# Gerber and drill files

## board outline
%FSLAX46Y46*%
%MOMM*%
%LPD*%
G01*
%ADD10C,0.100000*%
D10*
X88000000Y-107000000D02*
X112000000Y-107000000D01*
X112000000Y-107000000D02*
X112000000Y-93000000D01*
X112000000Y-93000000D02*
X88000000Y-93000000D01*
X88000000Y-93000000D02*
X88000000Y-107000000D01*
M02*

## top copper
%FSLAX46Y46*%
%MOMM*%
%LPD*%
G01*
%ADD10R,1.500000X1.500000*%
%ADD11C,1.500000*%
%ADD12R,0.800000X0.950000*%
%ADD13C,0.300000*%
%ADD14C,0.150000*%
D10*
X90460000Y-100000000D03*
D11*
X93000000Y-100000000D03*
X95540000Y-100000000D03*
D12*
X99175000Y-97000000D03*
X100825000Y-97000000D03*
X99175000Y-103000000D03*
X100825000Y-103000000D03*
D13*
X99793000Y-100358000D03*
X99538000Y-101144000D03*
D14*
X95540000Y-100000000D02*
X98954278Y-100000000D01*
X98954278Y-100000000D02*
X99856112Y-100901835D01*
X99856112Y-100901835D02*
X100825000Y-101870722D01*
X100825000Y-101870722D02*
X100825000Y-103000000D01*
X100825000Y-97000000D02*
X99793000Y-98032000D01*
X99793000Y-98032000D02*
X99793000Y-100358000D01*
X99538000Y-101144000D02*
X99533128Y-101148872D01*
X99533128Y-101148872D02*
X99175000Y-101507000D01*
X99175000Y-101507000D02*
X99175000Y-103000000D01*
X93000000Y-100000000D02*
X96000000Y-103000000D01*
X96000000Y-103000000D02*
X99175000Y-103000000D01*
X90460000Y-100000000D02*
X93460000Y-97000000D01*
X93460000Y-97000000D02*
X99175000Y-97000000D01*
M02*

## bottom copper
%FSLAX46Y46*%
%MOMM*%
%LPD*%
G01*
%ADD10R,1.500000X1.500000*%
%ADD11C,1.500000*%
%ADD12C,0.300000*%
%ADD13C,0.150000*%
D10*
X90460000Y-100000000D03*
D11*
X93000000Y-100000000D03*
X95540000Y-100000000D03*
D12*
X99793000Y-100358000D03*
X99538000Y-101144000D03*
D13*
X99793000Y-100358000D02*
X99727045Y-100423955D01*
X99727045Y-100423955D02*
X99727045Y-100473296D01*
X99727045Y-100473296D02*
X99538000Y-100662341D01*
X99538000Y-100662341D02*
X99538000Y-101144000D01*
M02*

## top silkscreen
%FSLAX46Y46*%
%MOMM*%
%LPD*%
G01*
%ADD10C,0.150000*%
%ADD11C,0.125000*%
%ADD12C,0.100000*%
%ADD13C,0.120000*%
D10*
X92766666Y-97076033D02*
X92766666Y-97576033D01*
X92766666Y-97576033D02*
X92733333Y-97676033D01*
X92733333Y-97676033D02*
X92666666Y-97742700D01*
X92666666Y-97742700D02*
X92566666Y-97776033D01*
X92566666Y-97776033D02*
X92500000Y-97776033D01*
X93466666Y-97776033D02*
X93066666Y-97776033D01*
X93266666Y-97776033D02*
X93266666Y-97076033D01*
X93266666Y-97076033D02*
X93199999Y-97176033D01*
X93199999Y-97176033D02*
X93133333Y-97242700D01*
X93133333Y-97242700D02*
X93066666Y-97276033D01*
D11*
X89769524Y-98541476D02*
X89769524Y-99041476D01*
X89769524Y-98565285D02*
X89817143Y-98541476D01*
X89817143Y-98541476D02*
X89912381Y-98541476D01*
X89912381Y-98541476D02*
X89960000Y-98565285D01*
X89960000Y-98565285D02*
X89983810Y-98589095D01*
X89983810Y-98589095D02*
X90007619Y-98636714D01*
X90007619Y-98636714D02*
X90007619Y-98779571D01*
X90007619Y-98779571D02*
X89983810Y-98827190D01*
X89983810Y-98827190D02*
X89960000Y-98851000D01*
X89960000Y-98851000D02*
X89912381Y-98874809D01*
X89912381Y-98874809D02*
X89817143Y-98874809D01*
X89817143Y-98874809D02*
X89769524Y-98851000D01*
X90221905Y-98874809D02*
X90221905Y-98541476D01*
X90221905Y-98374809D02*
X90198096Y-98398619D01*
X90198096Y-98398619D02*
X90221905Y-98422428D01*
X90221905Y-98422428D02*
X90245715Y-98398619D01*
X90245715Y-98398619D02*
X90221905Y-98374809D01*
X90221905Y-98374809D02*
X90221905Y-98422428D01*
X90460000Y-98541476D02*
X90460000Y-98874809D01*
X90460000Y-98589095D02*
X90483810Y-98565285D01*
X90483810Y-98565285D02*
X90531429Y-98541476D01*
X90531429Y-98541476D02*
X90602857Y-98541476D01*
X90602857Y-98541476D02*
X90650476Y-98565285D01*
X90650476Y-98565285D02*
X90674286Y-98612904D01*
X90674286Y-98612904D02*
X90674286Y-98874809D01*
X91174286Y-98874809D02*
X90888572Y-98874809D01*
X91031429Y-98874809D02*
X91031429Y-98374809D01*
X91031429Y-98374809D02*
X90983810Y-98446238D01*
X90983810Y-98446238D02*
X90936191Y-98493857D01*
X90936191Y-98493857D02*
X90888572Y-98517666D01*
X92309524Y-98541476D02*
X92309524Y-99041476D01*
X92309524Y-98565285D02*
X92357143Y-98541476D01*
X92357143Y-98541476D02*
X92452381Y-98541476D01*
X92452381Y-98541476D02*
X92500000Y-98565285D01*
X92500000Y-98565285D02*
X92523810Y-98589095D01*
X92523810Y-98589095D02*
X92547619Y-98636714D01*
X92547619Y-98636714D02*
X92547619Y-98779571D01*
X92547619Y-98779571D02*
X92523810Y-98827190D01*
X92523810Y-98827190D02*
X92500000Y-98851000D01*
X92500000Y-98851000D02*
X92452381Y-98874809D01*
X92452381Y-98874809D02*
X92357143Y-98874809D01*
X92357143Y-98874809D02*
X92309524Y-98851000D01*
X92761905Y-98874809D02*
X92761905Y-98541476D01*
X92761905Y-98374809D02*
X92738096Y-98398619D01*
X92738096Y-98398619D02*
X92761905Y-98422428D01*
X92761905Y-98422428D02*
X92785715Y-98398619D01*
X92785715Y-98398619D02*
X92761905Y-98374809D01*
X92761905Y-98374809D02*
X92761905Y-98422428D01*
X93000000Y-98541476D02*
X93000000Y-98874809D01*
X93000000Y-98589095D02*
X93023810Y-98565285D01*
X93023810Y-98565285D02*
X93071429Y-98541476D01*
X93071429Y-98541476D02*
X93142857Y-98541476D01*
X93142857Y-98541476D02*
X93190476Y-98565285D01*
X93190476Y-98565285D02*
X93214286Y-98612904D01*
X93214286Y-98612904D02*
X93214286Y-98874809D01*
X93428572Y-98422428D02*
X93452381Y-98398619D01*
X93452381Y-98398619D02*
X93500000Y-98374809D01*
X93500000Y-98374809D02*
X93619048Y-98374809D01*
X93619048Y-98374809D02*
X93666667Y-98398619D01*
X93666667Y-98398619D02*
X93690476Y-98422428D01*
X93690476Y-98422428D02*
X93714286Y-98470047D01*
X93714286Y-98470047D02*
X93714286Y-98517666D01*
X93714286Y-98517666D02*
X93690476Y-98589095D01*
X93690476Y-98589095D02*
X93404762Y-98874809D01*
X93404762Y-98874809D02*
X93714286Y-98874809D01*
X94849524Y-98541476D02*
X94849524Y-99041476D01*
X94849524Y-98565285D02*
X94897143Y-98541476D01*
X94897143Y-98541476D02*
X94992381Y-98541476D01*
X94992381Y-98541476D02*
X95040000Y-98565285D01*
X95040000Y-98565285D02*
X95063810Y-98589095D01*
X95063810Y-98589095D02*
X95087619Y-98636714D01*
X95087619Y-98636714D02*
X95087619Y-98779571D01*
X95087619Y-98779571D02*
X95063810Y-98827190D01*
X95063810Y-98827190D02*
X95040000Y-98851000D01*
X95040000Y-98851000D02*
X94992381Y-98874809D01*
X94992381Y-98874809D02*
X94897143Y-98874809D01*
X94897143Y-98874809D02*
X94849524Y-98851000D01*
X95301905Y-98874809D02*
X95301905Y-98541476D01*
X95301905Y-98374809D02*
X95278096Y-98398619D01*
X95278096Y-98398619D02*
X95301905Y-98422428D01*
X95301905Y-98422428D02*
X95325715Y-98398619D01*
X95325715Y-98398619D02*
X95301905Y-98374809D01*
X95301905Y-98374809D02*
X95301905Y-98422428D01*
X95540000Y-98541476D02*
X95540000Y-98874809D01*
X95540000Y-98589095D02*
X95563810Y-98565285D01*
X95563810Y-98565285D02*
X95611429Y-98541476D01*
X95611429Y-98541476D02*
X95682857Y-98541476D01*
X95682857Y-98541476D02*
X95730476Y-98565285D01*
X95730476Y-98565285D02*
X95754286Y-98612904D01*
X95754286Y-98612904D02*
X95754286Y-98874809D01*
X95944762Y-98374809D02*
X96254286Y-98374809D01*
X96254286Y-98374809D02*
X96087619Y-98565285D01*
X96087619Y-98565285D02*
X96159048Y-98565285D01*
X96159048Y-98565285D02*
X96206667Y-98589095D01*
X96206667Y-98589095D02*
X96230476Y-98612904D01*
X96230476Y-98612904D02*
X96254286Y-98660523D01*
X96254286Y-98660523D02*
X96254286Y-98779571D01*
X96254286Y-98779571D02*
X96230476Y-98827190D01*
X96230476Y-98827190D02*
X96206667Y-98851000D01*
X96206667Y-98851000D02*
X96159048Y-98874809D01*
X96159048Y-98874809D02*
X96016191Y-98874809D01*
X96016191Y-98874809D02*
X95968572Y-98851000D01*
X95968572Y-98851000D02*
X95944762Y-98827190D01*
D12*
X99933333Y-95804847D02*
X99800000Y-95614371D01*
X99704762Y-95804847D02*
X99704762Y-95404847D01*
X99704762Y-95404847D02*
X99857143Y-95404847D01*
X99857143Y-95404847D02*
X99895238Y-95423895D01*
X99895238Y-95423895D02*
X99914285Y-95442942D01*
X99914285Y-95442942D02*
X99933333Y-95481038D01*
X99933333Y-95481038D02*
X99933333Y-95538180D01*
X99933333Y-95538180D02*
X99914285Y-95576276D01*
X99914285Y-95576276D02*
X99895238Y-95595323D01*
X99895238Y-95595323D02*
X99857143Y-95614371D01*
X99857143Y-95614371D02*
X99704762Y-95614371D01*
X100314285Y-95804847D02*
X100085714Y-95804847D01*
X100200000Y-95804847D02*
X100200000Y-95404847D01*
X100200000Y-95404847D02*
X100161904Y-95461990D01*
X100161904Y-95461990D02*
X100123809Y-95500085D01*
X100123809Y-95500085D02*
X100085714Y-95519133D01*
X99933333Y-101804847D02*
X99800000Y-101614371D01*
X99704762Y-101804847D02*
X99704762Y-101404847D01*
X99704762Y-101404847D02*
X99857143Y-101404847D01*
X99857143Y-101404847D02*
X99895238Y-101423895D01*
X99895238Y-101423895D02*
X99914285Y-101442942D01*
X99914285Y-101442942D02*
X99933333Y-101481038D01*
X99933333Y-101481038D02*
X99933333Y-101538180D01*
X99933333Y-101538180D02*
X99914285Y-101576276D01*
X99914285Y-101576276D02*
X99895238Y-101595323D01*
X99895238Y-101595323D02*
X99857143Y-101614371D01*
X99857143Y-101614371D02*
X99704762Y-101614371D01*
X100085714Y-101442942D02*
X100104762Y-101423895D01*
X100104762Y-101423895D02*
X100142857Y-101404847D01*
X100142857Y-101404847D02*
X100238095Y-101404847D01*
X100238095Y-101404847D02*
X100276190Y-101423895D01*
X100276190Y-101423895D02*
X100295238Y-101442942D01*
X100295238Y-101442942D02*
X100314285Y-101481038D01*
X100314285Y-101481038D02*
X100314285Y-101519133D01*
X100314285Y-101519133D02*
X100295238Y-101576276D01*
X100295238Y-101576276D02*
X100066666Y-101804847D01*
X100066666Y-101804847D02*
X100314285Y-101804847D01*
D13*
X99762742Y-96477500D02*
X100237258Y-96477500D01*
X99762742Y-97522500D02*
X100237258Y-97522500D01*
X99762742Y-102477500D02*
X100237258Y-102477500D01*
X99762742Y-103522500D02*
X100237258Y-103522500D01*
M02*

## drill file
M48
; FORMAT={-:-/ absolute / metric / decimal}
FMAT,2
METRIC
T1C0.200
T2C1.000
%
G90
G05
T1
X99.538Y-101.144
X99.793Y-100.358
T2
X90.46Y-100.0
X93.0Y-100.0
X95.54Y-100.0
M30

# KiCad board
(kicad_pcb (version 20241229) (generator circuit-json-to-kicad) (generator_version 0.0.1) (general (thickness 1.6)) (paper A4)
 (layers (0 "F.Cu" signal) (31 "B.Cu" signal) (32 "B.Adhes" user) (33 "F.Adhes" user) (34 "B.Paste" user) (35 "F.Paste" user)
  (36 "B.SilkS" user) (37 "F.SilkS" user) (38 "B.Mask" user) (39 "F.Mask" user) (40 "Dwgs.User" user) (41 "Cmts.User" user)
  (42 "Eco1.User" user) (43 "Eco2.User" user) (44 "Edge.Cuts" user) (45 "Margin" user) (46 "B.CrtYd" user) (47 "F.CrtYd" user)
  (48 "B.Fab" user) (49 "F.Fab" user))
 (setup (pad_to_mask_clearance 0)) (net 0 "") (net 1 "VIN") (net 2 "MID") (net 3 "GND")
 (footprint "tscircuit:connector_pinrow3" (layer F.Cu) (at 93 100 0)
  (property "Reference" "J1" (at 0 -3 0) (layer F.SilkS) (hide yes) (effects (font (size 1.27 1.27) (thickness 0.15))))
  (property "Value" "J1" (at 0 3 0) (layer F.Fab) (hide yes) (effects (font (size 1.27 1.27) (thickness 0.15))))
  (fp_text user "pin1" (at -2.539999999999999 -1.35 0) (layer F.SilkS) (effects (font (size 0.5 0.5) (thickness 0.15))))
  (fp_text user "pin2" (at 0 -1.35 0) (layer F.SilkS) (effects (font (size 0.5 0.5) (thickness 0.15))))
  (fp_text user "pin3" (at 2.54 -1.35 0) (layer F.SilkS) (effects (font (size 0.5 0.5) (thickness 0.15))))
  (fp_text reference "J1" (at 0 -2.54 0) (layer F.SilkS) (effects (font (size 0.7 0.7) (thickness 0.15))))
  (pad "1" thru_hole rect (at -2.539999999999999 0 0) (size 1.5 1.5) (drill 1) (layers *.Cu *.Mask) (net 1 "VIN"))
  (pad "2" thru_hole circle (at 0 0 0) (size 1.5 1.5) (drill 1) (layers *.Cu *.Mask) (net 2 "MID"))
  (pad "3" thru_hole circle (at 2.54 0 0) (size 1.5 1.5) (drill 1) (layers *.Cu *.Mask) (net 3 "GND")))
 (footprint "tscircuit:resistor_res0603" (layer F.Cu) (at 100 97 0)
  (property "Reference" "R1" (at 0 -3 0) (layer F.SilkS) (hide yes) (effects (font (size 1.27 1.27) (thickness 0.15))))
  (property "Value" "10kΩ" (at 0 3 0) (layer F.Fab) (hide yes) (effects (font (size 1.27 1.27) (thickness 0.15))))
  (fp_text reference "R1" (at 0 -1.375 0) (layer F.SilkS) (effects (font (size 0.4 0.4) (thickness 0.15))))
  (fp_line (start -0.237258 -0.5225) (end 0.237258 -0.5225) (stroke (width 0.12) (type default)) (layer F.SilkS))
  (fp_line (start -0.237258 0.5225) (end 0.237258 0.5225) (stroke (width 0.12) (type default)) (layer F.SilkS))
  (pad "1" smd rect (at -0.825 0 0) (size 0.8 0.95) (layers F.Cu F.Mask) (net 1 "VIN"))
  (pad "2" smd rect (at 0.825 0 0) (size 0.8 0.95) (layers F.Cu F.Mask) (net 2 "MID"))
  (pad "" smd rect (at -0.825 0 0) (size 0.5599999999999999 0.6649999999999999) (layers F.Paste))
  (pad "" smd rect (at 0.825 0 0) (size 0.5599999999999999 0.6649999999999999) (layers F.Paste)))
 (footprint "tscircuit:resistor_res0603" (layer F.Cu) (at 100 103 0)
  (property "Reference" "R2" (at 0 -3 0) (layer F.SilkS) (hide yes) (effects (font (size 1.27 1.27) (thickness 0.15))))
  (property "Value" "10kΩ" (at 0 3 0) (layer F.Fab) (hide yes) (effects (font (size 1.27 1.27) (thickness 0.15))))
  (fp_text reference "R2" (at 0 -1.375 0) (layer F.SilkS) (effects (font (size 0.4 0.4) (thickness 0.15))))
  (fp_line (start -0.237258 -0.5225) (end 0.237258 -0.5225) (stroke (width 0.12) (type default)) (layer F.SilkS))
  (fp_line (start -0.237258 0.5225) (end 0.237258 0.5225) (stroke (width 0.12) (type default)) (layer F.SilkS))
  (pad "1" smd rect (at -0.825 0 0) (size 0.8 0.95) (layers F.Cu F.Mask) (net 2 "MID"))
  (pad "2" smd rect (at 0.825 0 0) (size 0.8 0.95) (layers F.Cu F.Mask) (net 3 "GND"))
  (pad "" smd rect (at -0.825 0 0) (size 0.5599999999999999 0.6649999999999999) (layers F.Paste))
  (pad "" smd rect (at 0.825 0 0) (size 0.5599999999999999 0.6649999999999999) (layers F.Paste)))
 (segment (start 95.54 100) (end 98.95427755765121 100) (width 0.15) (layer F.Cu) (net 3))
 (segment (start 98.95427755765121 100) (end 99.8561121118583 100.90183455420707) (width 0.15) (layer F.Cu) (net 3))
 (segment (start 99.8561121118583 100.90183455420707) (end 100.825 101.87072244234878) (width 0.15) (layer F.Cu) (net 3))
 (segment (start 100.825 101.87072244234878) (end 100.825 103) (width 0.15) (layer F.Cu) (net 3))
 (segment (start 100.825 97) (end 99.793 98.032) (width 0.15) (layer F.Cu) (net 2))
 (segment (start 99.793 98.032) (end 99.793 100.358) (width 0.15) (layer F.Cu) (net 2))
 (segment (start 99.793 100.358) (end 99.72704546466728 100.42395453533271) (width 0.15) (layer B.Cu) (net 2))
 (segment (start 99.72704546466728 100.42395453533271) (end 99.72704546466728 100.47329557476104) (width 0.15) (layer B.Cu) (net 2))
 (segment (start 99.72704546466728 100.47329557476104) (end 99.538 100.66234103942833) (width 0.15) (layer B.Cu) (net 2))
 (segment (start 99.538 100.66234103942833) (end 99.538 101.144) (width 0.15) (layer B.Cu) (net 2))
 (segment (start 99.538 101.144) (end 99.53312750305507 101.14887249694492) (width 0.15) (layer F.Cu) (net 2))
 (segment (start 99.53312750305507 101.14887249694492) (end 99.175 101.507) (width 0.15) (layer F.Cu) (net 2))
 (segment (start 99.175 101.507) (end 99.175 103) (width 0.15) (layer F.Cu) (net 2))
 (segment (start 93 100) (end 96 103) (width 0.15) (layer F.Cu) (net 2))
 (segment (start 96 103) (end 99.175 103) (width 0.15) (layer F.Cu) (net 2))
 (segment (start 90.46000000000001 100) (end 93.46000000000001 97) (width 0.15) (layer F.Cu) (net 1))
 (segment (start 93.46000000000001 97) (end 99.175 97) (width 0.15) (layer F.Cu) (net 1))
 (gr_line (start 88 107) (end 112 107) (width 0.1) (layer Edge.Cuts))
 (gr_line (start 112 107) (end 112 93) (width 0.1) (layer Edge.Cuts))
 (gr_line (start 112 93) (end 88 93) (width 0.1) (layer Edge.Cuts))
 (gr_line (start 88 93) (end 88 107) (width 0.1) (layer Edge.Cuts))
 (via (at 99.793 100.358) (size 0.3) (drill 0.2) (layers F.Cu B.Cu) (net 2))
 (via (at 99.538 101.144) (size 0.3) (drill 0.2) (layers F.Cu B.Cu) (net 2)))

